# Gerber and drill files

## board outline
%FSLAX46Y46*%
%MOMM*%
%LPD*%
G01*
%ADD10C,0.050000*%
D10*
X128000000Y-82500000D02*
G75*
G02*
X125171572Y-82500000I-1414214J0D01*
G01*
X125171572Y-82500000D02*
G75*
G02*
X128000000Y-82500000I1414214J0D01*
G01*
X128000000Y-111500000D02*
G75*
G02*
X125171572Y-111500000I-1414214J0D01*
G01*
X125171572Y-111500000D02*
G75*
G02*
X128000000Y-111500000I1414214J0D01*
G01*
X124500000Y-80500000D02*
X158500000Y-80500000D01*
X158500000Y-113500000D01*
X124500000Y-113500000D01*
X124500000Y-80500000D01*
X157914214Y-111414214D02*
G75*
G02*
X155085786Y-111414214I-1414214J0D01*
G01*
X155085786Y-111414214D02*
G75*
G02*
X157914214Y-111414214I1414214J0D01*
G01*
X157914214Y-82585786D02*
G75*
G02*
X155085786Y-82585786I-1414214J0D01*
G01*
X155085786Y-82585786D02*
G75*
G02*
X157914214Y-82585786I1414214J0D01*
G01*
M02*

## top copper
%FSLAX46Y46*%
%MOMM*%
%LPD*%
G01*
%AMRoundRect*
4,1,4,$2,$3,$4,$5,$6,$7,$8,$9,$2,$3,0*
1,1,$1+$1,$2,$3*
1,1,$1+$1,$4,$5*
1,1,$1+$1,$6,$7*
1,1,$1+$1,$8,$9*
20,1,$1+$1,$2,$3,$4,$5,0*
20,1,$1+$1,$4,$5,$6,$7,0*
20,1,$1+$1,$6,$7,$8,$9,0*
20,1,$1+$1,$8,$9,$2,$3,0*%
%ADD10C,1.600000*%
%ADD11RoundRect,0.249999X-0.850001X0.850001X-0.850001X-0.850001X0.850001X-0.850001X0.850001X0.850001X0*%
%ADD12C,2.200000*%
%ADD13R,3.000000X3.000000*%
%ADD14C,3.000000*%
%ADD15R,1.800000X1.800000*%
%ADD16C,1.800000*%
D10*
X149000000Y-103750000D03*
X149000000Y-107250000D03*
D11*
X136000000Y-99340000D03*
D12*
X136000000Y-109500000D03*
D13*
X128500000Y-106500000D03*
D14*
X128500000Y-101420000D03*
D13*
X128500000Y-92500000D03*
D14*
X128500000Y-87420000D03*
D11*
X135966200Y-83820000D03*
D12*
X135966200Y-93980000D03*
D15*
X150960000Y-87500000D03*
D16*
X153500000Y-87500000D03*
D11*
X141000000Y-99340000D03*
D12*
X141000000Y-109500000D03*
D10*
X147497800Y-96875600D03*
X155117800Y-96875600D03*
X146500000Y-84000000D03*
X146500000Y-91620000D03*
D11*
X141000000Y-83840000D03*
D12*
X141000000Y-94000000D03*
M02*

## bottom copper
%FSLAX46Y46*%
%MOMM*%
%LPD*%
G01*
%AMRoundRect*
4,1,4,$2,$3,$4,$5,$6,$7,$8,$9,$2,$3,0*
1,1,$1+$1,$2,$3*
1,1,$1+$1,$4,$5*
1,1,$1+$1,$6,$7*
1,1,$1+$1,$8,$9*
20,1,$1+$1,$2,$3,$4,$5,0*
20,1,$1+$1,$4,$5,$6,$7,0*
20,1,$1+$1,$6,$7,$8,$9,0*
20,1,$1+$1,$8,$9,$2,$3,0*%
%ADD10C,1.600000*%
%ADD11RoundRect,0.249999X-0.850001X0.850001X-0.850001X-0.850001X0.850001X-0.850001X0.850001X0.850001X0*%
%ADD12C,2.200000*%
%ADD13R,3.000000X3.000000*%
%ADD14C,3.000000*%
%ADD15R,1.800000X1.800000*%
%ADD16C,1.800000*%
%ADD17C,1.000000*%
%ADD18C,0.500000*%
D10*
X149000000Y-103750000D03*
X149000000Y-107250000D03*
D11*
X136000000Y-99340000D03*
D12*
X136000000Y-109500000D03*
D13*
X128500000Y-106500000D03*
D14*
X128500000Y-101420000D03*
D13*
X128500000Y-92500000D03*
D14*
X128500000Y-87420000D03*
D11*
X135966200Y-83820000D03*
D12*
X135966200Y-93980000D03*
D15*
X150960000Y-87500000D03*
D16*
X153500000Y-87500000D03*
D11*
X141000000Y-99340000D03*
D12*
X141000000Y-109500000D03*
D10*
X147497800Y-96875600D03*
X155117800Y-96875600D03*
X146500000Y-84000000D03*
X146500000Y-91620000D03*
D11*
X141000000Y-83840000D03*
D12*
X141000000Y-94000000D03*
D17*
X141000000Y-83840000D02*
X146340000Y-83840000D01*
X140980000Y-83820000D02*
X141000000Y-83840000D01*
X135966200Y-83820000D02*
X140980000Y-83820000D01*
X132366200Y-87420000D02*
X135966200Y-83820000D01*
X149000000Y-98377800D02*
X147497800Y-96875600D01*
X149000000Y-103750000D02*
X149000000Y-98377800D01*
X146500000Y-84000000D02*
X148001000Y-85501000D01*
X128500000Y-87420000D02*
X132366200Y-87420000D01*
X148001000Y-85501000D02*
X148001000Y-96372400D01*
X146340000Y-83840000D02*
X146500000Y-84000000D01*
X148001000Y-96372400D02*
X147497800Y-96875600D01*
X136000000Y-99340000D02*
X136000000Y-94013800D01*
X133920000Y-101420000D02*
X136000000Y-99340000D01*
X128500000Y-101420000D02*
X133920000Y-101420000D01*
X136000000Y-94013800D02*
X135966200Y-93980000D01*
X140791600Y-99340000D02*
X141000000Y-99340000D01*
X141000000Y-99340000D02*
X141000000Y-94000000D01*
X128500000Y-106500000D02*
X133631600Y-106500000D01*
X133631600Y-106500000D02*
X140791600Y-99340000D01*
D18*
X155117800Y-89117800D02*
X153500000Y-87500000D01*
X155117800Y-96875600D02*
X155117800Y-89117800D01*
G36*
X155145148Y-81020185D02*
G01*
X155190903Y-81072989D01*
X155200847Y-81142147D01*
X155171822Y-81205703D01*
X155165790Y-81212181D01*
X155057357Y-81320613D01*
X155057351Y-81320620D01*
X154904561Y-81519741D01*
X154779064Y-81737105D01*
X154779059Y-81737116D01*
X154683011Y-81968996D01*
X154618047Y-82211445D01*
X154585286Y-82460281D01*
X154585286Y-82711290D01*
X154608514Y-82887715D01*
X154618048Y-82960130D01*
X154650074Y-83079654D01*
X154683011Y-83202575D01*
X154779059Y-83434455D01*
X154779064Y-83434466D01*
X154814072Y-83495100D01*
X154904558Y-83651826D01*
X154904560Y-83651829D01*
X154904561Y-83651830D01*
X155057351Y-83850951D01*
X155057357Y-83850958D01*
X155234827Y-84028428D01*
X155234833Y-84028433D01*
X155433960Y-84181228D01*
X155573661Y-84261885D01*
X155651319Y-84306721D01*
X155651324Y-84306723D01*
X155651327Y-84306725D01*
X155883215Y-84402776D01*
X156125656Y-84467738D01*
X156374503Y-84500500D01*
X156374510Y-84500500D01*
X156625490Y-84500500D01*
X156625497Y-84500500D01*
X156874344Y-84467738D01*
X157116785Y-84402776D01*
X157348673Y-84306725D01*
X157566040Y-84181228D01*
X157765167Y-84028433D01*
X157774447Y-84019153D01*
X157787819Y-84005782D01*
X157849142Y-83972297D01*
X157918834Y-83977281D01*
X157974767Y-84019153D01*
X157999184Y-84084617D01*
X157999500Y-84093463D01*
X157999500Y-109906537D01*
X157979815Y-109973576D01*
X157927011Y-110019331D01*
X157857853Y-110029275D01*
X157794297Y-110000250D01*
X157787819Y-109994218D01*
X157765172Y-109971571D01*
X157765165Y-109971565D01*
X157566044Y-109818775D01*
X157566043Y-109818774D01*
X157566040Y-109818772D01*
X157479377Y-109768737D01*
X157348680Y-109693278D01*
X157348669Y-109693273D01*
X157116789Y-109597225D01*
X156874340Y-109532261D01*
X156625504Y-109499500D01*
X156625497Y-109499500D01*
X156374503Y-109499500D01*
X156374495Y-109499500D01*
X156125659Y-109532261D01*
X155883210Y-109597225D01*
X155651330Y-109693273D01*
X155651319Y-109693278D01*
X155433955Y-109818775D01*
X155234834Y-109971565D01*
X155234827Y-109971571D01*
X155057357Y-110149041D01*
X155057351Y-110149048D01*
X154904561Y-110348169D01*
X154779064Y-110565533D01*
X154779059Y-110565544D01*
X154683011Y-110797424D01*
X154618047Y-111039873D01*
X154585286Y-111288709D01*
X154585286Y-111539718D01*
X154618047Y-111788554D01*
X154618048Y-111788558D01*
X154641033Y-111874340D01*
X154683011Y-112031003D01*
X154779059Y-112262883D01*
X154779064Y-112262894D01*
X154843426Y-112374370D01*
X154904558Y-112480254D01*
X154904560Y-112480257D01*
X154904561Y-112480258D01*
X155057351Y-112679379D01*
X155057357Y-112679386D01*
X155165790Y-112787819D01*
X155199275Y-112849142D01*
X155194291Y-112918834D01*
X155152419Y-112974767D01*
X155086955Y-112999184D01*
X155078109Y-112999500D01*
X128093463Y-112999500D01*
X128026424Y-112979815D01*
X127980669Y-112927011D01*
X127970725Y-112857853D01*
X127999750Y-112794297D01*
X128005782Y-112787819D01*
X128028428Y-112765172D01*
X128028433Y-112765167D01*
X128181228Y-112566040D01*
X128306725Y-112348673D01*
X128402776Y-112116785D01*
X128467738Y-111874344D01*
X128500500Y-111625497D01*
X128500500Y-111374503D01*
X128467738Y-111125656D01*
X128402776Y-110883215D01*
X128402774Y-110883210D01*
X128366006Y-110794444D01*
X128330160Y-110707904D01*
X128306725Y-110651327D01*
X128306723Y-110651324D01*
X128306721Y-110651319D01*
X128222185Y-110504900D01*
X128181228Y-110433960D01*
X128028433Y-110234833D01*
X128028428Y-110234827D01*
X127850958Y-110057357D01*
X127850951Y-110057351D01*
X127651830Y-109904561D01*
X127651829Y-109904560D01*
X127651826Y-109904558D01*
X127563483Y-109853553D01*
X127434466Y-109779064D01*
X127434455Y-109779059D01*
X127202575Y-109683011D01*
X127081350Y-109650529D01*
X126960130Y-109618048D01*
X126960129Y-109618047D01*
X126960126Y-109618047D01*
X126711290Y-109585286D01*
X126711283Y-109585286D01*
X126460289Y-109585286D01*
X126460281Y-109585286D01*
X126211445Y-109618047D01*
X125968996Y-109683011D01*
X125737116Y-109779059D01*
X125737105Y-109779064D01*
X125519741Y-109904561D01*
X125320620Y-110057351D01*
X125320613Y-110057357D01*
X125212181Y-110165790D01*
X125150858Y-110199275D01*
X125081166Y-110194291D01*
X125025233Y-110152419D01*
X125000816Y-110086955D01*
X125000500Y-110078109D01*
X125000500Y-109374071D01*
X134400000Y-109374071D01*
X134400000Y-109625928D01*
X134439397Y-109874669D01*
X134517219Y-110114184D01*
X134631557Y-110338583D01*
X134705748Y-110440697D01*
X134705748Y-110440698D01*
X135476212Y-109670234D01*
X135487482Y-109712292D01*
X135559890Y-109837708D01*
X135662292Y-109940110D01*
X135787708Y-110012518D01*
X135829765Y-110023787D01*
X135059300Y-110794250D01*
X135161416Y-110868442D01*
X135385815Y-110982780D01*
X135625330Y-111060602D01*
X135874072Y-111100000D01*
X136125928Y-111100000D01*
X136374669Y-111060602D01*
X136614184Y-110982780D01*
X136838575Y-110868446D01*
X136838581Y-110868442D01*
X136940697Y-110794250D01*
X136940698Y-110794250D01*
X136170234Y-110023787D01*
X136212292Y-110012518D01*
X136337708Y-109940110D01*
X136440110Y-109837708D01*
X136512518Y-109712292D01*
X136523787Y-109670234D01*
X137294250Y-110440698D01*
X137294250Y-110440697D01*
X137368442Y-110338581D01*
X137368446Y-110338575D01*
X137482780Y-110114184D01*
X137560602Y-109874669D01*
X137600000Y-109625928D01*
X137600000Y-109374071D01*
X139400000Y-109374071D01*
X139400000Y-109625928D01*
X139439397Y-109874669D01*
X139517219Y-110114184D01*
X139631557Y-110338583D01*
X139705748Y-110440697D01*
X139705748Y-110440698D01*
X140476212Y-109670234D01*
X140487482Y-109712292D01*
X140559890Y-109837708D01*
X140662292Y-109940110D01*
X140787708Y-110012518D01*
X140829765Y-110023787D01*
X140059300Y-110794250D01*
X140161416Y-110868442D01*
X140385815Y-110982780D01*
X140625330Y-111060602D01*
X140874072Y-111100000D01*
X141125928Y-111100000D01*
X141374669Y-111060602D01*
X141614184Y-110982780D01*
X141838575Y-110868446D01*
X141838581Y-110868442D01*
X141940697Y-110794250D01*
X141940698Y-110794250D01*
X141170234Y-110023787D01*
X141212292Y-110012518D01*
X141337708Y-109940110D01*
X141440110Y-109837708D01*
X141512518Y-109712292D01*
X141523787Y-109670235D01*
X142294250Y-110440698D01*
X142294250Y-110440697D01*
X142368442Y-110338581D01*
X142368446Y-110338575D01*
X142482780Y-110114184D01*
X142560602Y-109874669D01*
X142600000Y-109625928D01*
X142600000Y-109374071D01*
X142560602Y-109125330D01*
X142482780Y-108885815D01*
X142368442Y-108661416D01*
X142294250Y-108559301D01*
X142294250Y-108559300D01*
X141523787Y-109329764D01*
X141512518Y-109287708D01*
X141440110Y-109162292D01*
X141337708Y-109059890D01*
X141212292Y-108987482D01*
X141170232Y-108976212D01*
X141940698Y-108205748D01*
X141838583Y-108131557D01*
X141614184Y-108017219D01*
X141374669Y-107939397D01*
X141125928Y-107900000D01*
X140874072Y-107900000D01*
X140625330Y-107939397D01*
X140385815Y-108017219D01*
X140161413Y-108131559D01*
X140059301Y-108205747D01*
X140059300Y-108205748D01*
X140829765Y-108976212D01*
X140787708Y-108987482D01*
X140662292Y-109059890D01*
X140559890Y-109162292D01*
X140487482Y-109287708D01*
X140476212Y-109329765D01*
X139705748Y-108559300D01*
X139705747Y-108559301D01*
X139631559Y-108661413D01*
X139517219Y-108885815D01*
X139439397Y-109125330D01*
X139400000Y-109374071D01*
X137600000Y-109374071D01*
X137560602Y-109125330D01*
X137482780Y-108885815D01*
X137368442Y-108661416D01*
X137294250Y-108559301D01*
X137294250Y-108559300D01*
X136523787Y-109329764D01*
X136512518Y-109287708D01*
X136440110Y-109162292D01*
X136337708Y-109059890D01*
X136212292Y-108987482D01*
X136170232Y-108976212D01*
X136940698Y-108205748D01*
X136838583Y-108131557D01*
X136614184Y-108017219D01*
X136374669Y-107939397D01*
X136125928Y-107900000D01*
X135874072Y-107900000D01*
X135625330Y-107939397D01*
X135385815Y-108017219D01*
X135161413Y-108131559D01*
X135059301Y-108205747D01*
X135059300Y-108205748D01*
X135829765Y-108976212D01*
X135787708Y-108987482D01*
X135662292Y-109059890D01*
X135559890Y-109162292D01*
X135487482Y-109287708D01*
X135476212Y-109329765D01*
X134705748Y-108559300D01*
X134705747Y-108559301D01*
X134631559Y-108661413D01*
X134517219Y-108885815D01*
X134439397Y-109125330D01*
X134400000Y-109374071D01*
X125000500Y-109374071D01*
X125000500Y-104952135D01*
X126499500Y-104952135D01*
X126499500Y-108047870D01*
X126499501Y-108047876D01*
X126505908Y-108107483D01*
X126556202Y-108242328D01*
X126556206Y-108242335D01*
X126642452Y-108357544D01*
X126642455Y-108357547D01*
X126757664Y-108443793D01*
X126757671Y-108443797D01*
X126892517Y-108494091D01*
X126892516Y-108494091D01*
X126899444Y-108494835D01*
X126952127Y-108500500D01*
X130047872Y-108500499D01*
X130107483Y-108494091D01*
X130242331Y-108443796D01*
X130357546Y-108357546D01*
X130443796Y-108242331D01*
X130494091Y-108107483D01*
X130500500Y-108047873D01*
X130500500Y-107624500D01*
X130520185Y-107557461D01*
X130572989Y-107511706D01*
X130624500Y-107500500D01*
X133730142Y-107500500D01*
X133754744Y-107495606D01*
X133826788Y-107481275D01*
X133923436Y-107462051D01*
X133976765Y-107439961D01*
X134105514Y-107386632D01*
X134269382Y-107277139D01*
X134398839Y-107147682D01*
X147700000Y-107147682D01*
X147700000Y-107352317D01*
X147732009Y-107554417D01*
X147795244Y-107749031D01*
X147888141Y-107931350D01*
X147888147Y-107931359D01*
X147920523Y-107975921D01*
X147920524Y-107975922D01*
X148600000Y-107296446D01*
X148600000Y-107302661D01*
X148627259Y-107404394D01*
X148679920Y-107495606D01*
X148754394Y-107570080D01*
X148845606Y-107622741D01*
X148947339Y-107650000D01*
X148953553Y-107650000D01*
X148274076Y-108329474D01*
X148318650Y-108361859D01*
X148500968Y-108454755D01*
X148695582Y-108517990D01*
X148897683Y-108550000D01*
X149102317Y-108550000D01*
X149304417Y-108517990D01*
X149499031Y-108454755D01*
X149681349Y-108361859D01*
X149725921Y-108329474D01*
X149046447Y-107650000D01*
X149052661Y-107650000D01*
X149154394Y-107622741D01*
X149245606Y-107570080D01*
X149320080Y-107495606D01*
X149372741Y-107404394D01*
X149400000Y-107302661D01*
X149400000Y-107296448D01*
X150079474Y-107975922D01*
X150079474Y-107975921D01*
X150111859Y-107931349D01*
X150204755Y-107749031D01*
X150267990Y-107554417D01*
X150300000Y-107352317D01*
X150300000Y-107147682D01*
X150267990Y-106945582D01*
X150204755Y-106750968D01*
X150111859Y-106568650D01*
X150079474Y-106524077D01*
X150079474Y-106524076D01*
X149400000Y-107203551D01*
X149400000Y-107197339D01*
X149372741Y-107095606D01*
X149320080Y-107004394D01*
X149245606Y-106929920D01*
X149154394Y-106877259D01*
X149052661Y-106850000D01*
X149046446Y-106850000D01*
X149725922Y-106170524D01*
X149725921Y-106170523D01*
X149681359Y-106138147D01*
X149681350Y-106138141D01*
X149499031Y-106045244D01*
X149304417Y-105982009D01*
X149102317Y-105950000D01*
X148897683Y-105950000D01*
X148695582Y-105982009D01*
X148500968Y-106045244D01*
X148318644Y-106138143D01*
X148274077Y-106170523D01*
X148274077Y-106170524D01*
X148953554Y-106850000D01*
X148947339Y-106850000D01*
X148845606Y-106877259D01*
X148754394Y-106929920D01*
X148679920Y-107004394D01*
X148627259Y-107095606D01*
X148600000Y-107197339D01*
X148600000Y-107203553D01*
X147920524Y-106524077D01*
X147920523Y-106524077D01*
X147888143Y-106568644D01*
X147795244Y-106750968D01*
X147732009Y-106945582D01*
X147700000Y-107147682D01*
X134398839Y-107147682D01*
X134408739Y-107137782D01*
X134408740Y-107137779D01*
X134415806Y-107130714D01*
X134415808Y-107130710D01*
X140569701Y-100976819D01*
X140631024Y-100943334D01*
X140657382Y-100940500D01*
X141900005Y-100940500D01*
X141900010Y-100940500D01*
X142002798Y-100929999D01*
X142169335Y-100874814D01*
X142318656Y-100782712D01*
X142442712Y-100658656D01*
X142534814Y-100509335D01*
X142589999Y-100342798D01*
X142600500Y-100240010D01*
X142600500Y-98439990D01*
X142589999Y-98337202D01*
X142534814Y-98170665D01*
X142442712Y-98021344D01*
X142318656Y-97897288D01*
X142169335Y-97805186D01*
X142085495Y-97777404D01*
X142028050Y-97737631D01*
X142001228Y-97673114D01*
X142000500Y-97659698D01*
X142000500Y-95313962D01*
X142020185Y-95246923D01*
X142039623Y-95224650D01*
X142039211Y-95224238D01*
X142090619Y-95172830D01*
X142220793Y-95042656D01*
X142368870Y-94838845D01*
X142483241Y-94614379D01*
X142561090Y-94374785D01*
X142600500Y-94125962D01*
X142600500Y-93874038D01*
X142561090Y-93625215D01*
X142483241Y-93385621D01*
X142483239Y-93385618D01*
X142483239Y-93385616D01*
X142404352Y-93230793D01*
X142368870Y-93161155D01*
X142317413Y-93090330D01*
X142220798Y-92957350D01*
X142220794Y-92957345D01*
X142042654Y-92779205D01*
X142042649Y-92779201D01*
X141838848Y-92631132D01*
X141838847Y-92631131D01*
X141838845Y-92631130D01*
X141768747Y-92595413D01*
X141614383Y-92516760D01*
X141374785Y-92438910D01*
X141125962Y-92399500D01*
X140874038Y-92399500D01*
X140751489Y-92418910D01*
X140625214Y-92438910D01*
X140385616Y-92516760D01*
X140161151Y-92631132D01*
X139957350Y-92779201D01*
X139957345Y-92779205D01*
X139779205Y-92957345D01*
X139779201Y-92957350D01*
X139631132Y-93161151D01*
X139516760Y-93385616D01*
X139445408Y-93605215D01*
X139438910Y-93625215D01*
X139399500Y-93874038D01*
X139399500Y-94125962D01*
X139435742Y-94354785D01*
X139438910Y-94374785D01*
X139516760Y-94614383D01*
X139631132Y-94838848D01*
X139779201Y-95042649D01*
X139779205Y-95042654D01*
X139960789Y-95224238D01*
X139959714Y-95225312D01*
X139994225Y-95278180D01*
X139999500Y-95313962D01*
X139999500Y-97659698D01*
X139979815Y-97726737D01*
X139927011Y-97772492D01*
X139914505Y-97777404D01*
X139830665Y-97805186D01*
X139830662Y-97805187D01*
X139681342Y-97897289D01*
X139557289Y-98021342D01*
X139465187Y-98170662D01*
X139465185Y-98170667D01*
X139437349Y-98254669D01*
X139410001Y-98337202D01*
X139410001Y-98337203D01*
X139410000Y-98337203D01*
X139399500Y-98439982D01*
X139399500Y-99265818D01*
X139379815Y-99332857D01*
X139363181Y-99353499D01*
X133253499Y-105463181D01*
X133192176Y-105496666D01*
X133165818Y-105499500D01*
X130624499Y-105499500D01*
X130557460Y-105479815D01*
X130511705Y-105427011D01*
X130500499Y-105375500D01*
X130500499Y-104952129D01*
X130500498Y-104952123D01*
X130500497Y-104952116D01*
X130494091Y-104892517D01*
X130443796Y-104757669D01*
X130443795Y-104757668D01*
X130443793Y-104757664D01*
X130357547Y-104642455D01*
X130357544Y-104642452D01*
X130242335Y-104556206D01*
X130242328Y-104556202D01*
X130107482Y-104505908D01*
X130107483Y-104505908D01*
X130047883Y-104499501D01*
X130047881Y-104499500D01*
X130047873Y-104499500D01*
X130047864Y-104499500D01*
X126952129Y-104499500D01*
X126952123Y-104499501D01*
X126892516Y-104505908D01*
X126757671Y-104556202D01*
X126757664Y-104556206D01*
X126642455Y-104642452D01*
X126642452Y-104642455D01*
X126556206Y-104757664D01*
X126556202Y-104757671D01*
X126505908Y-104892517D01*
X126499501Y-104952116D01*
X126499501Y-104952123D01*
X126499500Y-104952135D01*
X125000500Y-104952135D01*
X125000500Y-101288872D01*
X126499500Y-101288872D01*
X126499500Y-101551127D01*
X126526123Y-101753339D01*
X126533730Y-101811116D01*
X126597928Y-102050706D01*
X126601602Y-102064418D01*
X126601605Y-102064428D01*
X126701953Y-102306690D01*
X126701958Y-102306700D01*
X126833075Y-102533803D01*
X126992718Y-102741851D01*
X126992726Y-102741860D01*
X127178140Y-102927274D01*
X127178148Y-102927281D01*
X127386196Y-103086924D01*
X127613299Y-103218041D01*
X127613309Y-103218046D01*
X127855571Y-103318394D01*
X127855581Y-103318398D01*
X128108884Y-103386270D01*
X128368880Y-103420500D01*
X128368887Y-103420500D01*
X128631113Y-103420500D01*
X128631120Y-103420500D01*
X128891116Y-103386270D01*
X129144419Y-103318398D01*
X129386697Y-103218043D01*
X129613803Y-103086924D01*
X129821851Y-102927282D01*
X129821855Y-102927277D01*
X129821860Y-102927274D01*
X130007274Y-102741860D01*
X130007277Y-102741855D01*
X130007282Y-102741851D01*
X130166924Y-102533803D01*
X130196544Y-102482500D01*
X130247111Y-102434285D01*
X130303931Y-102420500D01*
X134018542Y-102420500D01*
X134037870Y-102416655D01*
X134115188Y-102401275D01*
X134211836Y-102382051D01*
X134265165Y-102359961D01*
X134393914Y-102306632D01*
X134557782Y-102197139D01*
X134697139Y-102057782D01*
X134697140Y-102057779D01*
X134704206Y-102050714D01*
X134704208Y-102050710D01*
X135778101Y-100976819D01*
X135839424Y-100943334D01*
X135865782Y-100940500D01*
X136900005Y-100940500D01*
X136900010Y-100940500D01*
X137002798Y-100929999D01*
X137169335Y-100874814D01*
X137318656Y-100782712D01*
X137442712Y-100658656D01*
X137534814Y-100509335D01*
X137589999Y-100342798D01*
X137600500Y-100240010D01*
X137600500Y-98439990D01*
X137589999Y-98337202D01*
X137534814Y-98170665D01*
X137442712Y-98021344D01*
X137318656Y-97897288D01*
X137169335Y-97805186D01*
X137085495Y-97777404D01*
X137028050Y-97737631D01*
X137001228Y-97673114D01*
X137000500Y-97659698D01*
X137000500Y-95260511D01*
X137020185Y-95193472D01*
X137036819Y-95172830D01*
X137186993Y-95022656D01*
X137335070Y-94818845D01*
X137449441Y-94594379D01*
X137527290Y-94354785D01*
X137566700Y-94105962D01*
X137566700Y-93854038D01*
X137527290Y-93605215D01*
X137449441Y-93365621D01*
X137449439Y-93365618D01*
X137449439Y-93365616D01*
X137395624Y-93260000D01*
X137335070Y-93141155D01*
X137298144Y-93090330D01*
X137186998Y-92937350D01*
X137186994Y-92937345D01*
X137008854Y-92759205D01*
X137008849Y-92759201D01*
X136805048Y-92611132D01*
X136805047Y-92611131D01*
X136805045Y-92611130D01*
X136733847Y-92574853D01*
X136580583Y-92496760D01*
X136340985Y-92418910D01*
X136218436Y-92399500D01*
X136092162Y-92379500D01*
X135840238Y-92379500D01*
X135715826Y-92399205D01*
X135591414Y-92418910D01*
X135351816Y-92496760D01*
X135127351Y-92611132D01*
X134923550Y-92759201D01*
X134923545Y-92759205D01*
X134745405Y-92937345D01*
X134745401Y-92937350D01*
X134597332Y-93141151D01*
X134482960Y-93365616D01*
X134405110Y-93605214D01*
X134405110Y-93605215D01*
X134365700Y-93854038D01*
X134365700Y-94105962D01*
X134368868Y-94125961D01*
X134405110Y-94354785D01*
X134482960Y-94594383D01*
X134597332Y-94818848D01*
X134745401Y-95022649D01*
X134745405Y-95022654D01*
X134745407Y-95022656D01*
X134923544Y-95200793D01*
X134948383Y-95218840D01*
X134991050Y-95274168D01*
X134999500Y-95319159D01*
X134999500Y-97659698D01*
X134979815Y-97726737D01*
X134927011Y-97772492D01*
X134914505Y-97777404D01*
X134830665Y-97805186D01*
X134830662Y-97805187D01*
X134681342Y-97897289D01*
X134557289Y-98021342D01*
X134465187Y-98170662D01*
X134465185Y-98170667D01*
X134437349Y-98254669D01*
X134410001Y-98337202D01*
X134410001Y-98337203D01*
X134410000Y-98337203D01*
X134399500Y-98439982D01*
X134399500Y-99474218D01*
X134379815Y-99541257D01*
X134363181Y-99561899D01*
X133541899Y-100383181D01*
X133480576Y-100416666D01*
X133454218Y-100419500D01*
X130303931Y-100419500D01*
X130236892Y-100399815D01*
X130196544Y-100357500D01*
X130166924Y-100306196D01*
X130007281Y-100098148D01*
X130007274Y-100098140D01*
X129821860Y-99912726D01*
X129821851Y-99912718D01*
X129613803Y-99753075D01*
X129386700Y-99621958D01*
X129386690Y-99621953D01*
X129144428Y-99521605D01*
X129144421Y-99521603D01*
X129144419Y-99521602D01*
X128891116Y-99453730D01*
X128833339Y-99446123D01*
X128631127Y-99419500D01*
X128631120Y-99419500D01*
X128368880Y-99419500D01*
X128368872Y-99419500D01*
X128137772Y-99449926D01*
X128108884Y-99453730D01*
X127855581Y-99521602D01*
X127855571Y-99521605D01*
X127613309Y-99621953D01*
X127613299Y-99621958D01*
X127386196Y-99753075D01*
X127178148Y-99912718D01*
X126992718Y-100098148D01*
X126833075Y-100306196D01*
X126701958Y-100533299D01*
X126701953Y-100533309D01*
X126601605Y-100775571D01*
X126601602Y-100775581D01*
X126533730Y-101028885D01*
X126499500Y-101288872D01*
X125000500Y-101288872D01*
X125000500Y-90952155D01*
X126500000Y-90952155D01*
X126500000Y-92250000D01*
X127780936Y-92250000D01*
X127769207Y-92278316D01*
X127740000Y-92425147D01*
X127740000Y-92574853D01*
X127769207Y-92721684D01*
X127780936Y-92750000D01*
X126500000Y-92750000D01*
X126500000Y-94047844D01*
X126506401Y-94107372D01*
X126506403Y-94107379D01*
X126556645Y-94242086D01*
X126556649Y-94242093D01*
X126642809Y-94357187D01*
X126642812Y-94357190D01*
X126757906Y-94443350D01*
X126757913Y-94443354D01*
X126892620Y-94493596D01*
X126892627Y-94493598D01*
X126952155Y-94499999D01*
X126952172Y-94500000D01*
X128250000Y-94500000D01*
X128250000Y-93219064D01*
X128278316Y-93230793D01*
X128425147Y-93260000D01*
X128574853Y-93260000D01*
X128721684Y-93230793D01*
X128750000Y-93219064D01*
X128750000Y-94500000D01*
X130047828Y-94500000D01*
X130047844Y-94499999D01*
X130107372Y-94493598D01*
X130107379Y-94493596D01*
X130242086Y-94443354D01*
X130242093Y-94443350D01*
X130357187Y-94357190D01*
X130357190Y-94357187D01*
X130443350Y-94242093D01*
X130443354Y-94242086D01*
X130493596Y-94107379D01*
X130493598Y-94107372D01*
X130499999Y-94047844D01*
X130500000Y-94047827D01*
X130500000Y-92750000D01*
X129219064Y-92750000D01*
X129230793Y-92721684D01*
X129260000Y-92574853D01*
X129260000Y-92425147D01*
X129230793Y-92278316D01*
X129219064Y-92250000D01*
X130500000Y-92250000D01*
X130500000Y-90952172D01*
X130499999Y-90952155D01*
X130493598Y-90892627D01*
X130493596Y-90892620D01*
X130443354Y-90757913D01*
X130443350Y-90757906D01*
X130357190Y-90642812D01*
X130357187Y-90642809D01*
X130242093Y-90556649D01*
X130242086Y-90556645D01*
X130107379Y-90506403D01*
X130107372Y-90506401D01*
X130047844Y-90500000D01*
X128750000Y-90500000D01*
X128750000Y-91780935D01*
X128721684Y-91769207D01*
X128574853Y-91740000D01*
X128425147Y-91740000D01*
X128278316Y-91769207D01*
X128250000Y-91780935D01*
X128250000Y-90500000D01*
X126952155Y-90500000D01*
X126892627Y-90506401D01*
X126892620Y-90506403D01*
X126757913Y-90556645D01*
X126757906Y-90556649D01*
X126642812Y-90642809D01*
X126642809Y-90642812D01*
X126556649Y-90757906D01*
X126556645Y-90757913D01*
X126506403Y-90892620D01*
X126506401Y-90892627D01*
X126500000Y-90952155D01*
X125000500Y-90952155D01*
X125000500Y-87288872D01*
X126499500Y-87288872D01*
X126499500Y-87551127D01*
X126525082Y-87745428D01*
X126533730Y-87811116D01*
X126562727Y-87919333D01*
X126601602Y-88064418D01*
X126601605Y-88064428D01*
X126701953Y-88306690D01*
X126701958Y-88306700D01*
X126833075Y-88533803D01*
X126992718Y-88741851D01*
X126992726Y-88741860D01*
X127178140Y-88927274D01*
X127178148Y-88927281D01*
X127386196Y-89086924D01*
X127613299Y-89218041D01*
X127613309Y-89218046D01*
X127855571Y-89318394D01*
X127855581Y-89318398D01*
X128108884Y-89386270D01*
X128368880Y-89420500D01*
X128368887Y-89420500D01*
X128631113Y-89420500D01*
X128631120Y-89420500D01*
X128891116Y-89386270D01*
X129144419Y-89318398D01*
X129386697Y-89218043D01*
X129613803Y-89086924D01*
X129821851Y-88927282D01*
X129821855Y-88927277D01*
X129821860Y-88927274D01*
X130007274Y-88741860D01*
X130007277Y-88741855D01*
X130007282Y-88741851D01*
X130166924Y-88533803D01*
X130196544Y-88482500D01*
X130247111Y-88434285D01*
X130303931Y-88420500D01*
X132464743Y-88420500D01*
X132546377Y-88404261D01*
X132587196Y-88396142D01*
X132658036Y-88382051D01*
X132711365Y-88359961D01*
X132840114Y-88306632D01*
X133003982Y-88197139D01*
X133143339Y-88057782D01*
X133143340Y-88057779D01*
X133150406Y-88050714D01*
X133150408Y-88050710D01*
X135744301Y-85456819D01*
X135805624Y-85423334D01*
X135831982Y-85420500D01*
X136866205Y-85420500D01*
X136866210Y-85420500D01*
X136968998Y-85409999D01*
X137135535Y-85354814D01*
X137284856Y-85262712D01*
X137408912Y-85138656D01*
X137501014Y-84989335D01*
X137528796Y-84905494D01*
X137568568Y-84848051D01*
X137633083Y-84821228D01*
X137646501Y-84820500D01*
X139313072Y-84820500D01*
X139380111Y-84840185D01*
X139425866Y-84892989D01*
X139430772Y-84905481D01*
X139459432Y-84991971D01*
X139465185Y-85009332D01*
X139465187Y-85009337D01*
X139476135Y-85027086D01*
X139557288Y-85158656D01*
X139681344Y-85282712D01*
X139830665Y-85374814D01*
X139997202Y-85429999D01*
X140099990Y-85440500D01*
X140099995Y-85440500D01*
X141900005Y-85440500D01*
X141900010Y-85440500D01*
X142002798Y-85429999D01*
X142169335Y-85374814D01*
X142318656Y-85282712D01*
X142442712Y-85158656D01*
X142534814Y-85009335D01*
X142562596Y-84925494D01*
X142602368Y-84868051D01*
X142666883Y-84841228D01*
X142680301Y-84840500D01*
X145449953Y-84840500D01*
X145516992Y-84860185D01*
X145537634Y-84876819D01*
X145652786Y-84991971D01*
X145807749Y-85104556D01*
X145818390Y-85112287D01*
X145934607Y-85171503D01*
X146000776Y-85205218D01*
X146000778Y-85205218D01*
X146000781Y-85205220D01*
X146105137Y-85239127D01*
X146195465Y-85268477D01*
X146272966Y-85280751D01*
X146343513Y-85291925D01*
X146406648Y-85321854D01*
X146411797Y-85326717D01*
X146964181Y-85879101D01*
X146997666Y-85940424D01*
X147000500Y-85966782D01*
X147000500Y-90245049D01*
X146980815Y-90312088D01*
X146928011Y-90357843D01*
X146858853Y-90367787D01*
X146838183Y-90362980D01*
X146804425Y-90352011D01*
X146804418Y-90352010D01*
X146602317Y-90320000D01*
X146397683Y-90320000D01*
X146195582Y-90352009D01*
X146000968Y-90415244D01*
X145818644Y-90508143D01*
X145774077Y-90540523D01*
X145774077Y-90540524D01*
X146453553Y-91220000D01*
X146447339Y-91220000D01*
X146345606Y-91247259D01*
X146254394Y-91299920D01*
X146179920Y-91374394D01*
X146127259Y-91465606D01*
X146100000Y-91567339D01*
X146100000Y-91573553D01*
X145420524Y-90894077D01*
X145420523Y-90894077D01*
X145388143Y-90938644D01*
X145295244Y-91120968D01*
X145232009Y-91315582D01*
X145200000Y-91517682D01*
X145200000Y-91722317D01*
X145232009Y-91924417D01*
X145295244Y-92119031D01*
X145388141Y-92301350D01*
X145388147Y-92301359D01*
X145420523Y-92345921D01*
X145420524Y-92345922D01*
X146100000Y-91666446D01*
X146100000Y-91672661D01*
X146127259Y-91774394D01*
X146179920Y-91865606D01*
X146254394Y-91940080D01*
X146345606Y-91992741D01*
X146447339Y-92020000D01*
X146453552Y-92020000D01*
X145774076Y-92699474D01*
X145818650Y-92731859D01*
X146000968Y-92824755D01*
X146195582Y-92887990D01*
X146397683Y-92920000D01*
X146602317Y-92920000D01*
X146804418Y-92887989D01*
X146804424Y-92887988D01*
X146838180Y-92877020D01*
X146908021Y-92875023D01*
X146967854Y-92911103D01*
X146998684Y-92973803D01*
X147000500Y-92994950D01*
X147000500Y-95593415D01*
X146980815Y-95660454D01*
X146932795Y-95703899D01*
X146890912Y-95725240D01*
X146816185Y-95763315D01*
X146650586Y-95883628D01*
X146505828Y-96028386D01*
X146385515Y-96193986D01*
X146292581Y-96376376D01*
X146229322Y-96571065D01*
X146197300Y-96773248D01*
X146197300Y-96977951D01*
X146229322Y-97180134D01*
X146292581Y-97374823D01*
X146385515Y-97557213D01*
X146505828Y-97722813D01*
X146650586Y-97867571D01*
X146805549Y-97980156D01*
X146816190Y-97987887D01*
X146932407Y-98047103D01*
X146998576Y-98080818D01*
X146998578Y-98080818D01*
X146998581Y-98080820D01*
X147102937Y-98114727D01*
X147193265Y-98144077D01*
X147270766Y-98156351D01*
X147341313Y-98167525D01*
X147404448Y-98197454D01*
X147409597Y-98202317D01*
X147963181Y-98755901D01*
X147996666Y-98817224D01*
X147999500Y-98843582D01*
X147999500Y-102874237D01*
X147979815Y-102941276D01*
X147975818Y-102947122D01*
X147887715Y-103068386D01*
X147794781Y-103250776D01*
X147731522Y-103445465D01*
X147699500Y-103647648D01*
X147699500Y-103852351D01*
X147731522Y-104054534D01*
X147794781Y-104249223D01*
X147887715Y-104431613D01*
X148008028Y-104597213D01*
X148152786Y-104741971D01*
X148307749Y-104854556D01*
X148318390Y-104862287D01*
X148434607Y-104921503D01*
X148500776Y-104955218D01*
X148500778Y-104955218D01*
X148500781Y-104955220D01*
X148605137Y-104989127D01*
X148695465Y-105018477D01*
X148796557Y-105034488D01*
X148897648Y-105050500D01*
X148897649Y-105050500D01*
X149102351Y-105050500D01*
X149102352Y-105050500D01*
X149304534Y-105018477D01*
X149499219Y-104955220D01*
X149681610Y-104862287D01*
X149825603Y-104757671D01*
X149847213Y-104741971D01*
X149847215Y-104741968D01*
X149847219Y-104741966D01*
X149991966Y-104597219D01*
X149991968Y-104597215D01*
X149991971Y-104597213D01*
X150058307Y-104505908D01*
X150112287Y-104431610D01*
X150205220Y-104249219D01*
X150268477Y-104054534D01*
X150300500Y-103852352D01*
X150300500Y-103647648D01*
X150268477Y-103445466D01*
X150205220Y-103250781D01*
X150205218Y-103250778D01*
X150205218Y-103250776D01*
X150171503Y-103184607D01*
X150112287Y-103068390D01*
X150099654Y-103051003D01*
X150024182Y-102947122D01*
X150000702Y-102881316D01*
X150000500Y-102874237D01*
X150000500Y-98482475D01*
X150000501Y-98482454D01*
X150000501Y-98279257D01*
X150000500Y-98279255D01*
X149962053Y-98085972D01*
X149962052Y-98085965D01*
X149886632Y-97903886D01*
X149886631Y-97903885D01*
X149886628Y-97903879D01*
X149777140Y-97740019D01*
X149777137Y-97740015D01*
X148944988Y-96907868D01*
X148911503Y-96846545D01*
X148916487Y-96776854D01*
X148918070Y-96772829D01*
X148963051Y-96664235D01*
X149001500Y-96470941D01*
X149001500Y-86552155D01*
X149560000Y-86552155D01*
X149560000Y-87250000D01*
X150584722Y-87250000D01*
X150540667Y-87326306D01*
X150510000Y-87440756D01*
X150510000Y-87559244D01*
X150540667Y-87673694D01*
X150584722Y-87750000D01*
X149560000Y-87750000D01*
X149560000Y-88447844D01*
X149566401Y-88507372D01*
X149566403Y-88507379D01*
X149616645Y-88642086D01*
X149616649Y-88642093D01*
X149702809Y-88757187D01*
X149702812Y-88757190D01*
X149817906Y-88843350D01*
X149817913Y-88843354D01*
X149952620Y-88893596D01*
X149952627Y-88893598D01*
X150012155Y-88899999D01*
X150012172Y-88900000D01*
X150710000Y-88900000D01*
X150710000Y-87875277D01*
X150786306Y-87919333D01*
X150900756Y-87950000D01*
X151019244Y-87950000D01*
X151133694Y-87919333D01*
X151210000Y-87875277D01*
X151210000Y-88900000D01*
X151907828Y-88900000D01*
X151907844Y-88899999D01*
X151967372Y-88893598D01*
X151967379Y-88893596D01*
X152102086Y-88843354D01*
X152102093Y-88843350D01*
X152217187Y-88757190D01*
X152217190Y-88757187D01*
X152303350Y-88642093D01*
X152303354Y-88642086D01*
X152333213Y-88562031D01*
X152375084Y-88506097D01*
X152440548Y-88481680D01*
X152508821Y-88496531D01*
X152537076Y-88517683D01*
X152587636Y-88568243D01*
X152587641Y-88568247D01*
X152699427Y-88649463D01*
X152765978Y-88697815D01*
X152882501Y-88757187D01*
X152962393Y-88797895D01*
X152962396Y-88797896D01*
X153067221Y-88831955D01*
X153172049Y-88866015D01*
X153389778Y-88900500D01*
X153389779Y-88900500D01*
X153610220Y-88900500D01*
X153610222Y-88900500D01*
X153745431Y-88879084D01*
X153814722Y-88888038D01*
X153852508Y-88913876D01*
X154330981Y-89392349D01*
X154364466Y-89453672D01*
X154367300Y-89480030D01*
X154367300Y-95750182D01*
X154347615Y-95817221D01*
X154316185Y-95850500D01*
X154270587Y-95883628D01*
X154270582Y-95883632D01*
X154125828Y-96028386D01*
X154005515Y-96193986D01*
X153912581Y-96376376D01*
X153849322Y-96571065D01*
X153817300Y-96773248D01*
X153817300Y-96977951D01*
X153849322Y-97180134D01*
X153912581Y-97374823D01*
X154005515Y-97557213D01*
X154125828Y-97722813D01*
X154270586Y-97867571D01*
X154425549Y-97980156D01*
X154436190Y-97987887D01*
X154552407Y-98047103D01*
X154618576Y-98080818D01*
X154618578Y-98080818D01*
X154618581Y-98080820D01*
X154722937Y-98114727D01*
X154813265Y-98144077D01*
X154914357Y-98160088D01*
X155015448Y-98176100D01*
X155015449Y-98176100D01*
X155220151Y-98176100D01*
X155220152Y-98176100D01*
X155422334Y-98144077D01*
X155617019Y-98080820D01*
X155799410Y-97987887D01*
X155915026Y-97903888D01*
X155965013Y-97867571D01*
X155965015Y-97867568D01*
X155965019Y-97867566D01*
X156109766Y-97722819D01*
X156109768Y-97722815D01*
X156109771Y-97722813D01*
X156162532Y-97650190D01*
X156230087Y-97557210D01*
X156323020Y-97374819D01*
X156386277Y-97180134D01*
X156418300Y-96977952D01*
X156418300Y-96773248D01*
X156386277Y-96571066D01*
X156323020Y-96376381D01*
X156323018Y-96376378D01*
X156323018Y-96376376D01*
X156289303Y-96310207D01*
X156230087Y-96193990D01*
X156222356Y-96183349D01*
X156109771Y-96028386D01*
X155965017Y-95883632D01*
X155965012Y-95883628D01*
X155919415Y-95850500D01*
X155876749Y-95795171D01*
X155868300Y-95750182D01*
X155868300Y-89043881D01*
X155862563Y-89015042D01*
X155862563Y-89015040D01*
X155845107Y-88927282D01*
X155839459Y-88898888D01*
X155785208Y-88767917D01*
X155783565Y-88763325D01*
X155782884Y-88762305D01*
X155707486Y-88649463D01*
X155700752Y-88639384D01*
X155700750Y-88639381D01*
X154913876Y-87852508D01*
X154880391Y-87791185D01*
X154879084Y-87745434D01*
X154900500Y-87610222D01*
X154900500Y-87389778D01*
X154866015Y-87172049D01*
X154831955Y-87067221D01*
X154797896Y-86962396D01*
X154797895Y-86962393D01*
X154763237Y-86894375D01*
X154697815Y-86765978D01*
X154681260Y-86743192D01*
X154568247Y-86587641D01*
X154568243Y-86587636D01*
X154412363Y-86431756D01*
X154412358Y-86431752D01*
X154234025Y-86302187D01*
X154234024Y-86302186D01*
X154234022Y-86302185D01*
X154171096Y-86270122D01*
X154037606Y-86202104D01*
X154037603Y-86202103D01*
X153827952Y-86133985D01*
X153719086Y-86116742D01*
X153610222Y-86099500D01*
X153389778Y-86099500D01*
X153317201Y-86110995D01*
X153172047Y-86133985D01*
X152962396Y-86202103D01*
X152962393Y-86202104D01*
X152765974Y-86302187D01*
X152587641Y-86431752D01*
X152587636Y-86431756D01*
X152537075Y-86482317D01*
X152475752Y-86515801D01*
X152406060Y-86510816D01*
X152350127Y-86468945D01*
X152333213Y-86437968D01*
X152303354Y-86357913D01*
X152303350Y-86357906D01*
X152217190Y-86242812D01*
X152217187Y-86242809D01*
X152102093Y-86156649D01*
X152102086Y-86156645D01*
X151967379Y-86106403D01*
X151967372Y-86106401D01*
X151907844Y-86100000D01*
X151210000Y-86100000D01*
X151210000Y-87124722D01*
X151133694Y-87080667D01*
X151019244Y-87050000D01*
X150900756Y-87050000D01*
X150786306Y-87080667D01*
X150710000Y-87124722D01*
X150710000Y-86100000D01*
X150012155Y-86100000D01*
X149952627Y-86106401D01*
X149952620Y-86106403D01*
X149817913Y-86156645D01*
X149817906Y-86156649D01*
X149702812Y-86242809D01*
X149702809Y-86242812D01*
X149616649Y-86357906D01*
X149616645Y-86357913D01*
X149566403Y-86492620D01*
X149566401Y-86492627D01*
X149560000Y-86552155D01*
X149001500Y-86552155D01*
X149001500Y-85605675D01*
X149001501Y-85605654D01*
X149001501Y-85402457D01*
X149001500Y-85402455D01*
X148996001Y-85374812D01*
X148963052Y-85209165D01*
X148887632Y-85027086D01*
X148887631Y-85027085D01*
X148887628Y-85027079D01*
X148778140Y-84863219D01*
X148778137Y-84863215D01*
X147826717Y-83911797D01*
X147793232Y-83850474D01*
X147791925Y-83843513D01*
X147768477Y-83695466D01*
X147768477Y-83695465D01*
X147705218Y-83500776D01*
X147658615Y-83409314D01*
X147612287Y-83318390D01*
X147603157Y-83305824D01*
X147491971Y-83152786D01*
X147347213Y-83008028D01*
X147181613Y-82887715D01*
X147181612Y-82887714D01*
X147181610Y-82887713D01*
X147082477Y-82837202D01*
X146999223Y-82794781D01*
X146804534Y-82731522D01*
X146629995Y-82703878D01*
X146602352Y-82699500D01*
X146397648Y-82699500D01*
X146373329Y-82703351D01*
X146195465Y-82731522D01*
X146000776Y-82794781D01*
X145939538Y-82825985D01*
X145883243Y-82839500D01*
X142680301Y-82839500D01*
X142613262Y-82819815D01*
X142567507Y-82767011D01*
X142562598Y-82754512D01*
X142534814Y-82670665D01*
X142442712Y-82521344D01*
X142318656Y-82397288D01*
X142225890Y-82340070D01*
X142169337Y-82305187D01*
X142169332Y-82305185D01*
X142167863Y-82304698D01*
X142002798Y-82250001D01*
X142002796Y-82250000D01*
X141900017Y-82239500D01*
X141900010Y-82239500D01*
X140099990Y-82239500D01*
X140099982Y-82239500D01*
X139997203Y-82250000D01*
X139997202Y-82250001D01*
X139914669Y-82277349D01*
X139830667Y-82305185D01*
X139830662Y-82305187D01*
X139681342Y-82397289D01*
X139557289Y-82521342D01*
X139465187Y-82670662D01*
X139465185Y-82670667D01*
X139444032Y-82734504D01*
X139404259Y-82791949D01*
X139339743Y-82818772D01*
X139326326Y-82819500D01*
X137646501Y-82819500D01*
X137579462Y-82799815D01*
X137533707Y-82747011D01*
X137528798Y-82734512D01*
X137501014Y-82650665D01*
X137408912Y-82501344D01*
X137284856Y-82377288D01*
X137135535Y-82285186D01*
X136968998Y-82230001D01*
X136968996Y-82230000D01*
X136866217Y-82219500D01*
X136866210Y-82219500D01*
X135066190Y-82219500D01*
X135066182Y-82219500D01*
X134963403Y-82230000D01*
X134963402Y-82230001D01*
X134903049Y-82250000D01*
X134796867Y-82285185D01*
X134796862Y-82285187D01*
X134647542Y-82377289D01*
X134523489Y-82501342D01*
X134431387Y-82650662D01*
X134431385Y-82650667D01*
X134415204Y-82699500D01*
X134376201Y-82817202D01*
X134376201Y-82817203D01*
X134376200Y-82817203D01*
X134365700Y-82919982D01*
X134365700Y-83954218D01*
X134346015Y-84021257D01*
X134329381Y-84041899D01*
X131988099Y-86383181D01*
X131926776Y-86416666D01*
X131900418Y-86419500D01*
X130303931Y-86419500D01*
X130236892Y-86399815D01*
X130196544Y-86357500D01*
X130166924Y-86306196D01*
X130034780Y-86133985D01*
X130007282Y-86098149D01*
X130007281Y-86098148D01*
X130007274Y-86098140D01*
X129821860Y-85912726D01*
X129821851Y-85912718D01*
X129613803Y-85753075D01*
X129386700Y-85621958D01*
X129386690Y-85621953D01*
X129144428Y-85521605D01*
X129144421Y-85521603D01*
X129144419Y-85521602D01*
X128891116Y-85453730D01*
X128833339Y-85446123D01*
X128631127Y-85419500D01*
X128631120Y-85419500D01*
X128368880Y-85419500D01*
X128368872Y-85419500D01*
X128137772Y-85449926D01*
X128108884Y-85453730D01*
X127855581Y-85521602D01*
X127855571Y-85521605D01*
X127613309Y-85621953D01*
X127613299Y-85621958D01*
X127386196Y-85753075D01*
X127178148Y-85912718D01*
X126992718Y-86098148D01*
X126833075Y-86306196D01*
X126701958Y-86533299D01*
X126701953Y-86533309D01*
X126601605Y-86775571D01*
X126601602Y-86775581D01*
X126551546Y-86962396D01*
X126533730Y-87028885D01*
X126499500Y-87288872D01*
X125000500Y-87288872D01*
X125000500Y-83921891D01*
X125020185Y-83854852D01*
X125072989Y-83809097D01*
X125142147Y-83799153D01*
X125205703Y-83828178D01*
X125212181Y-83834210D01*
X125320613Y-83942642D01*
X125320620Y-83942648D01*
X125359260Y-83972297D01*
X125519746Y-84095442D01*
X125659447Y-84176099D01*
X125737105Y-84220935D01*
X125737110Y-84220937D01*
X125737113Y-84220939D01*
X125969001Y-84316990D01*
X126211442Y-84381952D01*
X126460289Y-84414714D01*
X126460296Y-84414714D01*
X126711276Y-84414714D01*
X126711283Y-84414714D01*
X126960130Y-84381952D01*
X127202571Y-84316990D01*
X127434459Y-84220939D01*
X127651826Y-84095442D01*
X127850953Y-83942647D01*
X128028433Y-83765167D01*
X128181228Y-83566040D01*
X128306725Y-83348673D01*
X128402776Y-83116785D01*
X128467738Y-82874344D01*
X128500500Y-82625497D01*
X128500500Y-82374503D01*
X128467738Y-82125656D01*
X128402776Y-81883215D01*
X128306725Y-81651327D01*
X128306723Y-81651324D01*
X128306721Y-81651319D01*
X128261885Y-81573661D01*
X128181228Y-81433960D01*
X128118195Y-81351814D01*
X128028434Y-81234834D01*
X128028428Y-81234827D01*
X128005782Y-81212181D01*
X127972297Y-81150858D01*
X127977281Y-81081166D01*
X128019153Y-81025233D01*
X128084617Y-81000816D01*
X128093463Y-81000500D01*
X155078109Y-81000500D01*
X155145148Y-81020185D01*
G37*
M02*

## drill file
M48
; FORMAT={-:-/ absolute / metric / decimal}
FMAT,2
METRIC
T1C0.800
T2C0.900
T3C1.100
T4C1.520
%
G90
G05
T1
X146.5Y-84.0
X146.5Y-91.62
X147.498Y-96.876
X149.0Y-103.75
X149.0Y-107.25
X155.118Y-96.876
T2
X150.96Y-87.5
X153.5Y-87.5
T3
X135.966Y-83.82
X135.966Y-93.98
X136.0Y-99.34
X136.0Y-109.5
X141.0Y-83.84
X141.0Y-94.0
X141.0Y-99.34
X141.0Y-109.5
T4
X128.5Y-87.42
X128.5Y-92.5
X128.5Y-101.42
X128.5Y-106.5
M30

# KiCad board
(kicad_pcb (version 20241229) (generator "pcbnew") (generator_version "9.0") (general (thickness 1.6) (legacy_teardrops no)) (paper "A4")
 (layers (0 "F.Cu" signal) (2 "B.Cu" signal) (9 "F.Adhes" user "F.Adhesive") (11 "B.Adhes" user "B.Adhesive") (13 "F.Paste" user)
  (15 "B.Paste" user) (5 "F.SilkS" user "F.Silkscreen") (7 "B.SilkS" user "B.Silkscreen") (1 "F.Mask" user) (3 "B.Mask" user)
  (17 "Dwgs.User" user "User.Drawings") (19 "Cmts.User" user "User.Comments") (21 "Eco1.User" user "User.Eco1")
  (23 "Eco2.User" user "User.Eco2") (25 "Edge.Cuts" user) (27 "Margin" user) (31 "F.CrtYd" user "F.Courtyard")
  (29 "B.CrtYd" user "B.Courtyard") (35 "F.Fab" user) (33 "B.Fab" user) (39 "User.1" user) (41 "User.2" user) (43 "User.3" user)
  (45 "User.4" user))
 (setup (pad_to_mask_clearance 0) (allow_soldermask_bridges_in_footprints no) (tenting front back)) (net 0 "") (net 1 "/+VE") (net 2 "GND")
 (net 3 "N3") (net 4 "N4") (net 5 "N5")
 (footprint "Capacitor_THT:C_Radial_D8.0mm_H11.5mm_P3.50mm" (layer "F.Cu") (at 149 103.75 -90)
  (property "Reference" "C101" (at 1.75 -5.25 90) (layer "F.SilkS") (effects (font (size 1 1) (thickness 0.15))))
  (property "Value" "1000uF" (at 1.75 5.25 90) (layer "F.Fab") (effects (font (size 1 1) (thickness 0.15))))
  (pad "1" thru_hole circle (at 0 0 270) (size 1.6 1.6) (drill 0.8) (layers "*.Cu" "*.Mask") (remove_unused_layers no) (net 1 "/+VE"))
  (pad "2" thru_hole circle (at 3.5 0 270) (size 1.6 1.6) (drill 0.8) (layers "*.Cu" "*.Mask") (remove_unused_layers no) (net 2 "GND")))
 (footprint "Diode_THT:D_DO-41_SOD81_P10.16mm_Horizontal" (layer "F.Cu") (at 136 99.34 -90)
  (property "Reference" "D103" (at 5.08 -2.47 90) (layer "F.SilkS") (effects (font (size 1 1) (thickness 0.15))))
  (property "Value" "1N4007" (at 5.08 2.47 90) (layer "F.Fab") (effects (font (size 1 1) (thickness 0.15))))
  (pad "1" thru_hole roundrect (at 0 0 270) (size 2.2 2.2) (drill 1.1) (layers "*.Cu" "*.Mask") (remove_unused_layers no)
   (roundrect_rratio 0.113636) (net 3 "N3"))
  (pad "2" thru_hole circle (at 10.16 0 270) (size 2.2 2.2) (drill 1.1) (layers "*.Cu" "*.Mask") (remove_unused_layers no) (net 2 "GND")))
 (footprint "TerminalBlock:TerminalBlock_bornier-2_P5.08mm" (layer "F.Cu") (at 128.5 106.5 90)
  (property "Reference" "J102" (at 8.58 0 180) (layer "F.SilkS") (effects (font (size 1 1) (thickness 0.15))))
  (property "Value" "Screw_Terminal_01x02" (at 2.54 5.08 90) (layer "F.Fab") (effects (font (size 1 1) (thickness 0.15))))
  (pad "1" thru_hole rect (at 0 0 90) (size 3 3) (drill 1.52) (layers "*.Cu" "*.Mask") (remove_unused_layers no) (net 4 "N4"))
  (pad "2" thru_hole circle (at 5.08 0 90) (size 3 3) (drill 1.52) (layers "*.Cu" "*.Mask") (remove_unused_layers no) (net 3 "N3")))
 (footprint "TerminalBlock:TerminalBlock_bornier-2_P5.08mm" (layer "F.Cu") (at 128.5 92.5 90)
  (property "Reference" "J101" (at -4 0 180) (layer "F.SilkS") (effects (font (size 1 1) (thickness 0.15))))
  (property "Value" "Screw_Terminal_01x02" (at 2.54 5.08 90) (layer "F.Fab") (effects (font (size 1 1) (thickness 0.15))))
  (pad "1" thru_hole rect (at 0 0 90) (size 3 3) (drill 1.52) (layers "*.Cu" "*.Mask") (remove_unused_layers no) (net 2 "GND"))
  (pad "2" thru_hole circle (at 5.08 0 90) (size 3 3) (drill 1.52) (layers "*.Cu" "*.Mask") (remove_unused_layers no) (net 1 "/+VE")))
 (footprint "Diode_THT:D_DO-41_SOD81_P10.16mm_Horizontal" (layer "F.Cu") (at 135.9662 83.82 -90)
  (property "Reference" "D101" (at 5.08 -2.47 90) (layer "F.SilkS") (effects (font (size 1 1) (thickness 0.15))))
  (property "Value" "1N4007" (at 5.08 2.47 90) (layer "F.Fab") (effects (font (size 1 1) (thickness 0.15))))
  (pad "1" thru_hole roundrect (at 0 0 270) (size 2.2 2.2) (drill 1.1) (layers "*.Cu" "*.Mask") (remove_unused_layers no)
   (roundrect_rratio 0.113636) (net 1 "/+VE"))
  (pad "2" thru_hole circle (at 10.16 0 270) (size 2.2 2.2) (drill 1.1) (layers "*.Cu" "*.Mask") (remove_unused_layers no) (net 3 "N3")))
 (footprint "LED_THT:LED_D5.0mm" (layer "F.Cu") (at 150.96 87.5)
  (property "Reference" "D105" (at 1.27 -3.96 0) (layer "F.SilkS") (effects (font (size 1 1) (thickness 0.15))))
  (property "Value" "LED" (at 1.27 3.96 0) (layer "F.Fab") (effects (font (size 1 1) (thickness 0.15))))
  (pad "1" thru_hole rect (at 0 0) (size 1.8 1.8) (drill 0.9) (layers "*.Cu" "*.Mask") (remove_unused_layers no) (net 2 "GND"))
  (pad "2" thru_hole circle (at 2.54 0) (size 1.8 1.8) (drill 0.9) (layers "*.Cu" "*.Mask") (remove_unused_layers no) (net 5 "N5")))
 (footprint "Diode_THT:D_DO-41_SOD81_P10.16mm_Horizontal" (layer "F.Cu") (at 141 99.34 -90)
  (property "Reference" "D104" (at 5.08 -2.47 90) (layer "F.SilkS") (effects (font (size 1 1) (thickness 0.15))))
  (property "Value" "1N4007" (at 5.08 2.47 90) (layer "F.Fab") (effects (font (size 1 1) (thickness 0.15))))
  (pad "1" thru_hole roundrect (at 0 0 270) (size 2.2 2.2) (drill 1.1) (layers "*.Cu" "*.Mask") (remove_unused_layers no)
   (roundrect_rratio 0.113636) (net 4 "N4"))
  (pad "2" thru_hole circle (at 10.16 0 270) (size 2.2 2.2) (drill 1.1) (layers "*.Cu" "*.Mask") (remove_unused_layers no) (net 2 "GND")))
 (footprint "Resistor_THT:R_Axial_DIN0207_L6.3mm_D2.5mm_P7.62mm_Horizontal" (layer "F.Cu") (at 147.4978 96.8756)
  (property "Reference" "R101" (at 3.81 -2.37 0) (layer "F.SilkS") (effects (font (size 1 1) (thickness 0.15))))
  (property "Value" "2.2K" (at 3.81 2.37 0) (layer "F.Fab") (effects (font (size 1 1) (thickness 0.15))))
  (pad "1" thru_hole circle (at 0 0) (size 1.6 1.6) (drill 0.8) (layers "*.Cu" "*.Mask") (remove_unused_layers no) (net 1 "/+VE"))
  (pad "2" thru_hole circle (at 7.62 0) (size 1.6 1.6) (drill 0.8) (layers "*.Cu" "*.Mask") (remove_unused_layers no) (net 5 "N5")))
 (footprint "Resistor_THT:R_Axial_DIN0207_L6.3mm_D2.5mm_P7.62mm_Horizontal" (layer "F.Cu") (at 146.5 84 -90)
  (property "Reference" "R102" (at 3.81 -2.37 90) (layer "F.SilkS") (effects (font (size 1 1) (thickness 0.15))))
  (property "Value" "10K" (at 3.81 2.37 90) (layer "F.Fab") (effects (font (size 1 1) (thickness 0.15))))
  (pad "1" thru_hole circle (at 0 0 270) (size 1.6 1.6) (drill 0.8) (layers "*.Cu" "*.Mask") (remove_unused_layers no) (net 1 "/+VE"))
  (pad "2" thru_hole circle (at 7.62 0 270) (size 1.6 1.6) (drill 0.8) (layers "*.Cu" "*.Mask") (remove_unused_layers no) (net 2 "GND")))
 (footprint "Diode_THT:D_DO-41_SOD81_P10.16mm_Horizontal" (layer "F.Cu") (at 141 83.84 -90)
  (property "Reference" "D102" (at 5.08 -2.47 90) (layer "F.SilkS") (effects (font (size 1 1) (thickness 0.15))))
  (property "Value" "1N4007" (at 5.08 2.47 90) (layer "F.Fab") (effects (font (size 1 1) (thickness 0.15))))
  (pad "1" thru_hole roundrect (at 0 0 270) (size 2.2 2.2) (drill 1.1) (layers "*.Cu" "*.Mask") (remove_unused_layers no)
   (roundrect_rratio 0.113636) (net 1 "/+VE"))
  (pad "2" thru_hole circle (at 10.16 0 270) (size 2.2 2.2) (drill 1.1) (layers "*.Cu" "*.Mask") (remove_unused_layers no) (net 4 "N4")))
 (gr_circle (center 126.585786 82.5) (end 127.585786 83.5) (stroke (width 0.05) (type default)) (fill no) (layer "Edge.Cuts"))
 (gr_circle (center 126.585786 111.5) (end 127.585786 112.5) (stroke (width 0.05) (type default)) (fill no) (layer "Edge.Cuts"))
 (gr_rect (start 124.5 80.5) (end 158.5 113.5) (stroke (width 0.05) (type default)) (fill no) (layer "Edge.Cuts"))
 (gr_circle (center 156.5 111.414214) (end 157.5 112.414214) (stroke (width 0.05) (type default)) (fill no) (layer "Edge.Cuts"))
 (gr_circle (center 156.5 82.585786) (end 157.5 83.585786) (stroke (width 0.05) (type default)) (fill no) (layer "Edge.Cuts"))
 (segment (start 141 83.84) (end 146.34 83.84) (width 1) (layer "B.Cu") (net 1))
 (segment (start 140.98 83.82) (end 141 83.84) (width 1) (layer "B.Cu") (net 1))
 (segment (start 135.9662 83.82) (end 140.98 83.82) (width 1) (layer "B.Cu") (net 1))
 (segment (start 132.3662 87.42) (end 135.9662 83.82) (width 1) (layer "B.Cu") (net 1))
 (segment (start 149 98.3778) (end 147.4978 96.8756) (width 1) (layer "B.Cu") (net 1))
 (segment (start 149 103.75) (end 149 98.3778) (width 1) (layer "B.Cu") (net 1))
 (segment (start 146.5 84) (end 148.001 85.501) (width 1) (layer "B.Cu") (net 1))
 (segment (start 128.5 87.42) (end 132.3662 87.42) (width 1) (layer "B.Cu") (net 1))
 (segment (start 148.001 85.501) (end 148.001 96.3724) (width 1) (layer "B.Cu") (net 1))
 (segment (start 146.34 83.84) (end 146.5 84) (width 1) (layer "B.Cu") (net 1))
 (segment (start 148.001 96.3724) (end 147.4978 96.8756) (width 1) (layer "B.Cu") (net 1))
 (segment (start 136 99.34) (end 136 94.0138) (width 1) (layer "B.Cu") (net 3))
 (segment (start 133.92 101.42) (end 136 99.34) (width 1) (layer "B.Cu") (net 3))
 (segment (start 128.5 101.42) (end 133.92 101.42) (width 1) (layer "B.Cu") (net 3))
 (segment (start 136 94.0138) (end 135.9662 93.98) (width 1) (layer "B.Cu") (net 3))
 (segment (start 140.7916 99.34) (end 141 99.34) (width 1) (layer "B.Cu") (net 4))
 (segment (start 141 99.34) (end 141 94) (width 1) (layer "B.Cu") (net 4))
 (segment (start 128.5 106.5) (end 133.6316 106.5) (width 1) (layer "B.Cu") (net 4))
 (segment (start 133.6316 106.5) (end 140.7916 99.34) (width 1) (layer "B.Cu") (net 4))
 (segment (start 155.1178 89.1178) (end 153.5 87.5) (width 0.5) (layer "B.Cu") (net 5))
 (segment (start 155.1178 96.8756) (end 155.1178 89.1178) (width 0.5) (layer "B.Cu") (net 5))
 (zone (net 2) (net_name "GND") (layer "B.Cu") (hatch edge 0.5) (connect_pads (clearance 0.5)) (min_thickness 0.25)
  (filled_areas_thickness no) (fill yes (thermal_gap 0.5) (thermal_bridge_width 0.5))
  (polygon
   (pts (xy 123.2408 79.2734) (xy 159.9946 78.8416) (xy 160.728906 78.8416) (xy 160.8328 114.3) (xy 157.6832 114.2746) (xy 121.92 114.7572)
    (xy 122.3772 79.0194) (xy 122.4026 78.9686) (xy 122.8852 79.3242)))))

